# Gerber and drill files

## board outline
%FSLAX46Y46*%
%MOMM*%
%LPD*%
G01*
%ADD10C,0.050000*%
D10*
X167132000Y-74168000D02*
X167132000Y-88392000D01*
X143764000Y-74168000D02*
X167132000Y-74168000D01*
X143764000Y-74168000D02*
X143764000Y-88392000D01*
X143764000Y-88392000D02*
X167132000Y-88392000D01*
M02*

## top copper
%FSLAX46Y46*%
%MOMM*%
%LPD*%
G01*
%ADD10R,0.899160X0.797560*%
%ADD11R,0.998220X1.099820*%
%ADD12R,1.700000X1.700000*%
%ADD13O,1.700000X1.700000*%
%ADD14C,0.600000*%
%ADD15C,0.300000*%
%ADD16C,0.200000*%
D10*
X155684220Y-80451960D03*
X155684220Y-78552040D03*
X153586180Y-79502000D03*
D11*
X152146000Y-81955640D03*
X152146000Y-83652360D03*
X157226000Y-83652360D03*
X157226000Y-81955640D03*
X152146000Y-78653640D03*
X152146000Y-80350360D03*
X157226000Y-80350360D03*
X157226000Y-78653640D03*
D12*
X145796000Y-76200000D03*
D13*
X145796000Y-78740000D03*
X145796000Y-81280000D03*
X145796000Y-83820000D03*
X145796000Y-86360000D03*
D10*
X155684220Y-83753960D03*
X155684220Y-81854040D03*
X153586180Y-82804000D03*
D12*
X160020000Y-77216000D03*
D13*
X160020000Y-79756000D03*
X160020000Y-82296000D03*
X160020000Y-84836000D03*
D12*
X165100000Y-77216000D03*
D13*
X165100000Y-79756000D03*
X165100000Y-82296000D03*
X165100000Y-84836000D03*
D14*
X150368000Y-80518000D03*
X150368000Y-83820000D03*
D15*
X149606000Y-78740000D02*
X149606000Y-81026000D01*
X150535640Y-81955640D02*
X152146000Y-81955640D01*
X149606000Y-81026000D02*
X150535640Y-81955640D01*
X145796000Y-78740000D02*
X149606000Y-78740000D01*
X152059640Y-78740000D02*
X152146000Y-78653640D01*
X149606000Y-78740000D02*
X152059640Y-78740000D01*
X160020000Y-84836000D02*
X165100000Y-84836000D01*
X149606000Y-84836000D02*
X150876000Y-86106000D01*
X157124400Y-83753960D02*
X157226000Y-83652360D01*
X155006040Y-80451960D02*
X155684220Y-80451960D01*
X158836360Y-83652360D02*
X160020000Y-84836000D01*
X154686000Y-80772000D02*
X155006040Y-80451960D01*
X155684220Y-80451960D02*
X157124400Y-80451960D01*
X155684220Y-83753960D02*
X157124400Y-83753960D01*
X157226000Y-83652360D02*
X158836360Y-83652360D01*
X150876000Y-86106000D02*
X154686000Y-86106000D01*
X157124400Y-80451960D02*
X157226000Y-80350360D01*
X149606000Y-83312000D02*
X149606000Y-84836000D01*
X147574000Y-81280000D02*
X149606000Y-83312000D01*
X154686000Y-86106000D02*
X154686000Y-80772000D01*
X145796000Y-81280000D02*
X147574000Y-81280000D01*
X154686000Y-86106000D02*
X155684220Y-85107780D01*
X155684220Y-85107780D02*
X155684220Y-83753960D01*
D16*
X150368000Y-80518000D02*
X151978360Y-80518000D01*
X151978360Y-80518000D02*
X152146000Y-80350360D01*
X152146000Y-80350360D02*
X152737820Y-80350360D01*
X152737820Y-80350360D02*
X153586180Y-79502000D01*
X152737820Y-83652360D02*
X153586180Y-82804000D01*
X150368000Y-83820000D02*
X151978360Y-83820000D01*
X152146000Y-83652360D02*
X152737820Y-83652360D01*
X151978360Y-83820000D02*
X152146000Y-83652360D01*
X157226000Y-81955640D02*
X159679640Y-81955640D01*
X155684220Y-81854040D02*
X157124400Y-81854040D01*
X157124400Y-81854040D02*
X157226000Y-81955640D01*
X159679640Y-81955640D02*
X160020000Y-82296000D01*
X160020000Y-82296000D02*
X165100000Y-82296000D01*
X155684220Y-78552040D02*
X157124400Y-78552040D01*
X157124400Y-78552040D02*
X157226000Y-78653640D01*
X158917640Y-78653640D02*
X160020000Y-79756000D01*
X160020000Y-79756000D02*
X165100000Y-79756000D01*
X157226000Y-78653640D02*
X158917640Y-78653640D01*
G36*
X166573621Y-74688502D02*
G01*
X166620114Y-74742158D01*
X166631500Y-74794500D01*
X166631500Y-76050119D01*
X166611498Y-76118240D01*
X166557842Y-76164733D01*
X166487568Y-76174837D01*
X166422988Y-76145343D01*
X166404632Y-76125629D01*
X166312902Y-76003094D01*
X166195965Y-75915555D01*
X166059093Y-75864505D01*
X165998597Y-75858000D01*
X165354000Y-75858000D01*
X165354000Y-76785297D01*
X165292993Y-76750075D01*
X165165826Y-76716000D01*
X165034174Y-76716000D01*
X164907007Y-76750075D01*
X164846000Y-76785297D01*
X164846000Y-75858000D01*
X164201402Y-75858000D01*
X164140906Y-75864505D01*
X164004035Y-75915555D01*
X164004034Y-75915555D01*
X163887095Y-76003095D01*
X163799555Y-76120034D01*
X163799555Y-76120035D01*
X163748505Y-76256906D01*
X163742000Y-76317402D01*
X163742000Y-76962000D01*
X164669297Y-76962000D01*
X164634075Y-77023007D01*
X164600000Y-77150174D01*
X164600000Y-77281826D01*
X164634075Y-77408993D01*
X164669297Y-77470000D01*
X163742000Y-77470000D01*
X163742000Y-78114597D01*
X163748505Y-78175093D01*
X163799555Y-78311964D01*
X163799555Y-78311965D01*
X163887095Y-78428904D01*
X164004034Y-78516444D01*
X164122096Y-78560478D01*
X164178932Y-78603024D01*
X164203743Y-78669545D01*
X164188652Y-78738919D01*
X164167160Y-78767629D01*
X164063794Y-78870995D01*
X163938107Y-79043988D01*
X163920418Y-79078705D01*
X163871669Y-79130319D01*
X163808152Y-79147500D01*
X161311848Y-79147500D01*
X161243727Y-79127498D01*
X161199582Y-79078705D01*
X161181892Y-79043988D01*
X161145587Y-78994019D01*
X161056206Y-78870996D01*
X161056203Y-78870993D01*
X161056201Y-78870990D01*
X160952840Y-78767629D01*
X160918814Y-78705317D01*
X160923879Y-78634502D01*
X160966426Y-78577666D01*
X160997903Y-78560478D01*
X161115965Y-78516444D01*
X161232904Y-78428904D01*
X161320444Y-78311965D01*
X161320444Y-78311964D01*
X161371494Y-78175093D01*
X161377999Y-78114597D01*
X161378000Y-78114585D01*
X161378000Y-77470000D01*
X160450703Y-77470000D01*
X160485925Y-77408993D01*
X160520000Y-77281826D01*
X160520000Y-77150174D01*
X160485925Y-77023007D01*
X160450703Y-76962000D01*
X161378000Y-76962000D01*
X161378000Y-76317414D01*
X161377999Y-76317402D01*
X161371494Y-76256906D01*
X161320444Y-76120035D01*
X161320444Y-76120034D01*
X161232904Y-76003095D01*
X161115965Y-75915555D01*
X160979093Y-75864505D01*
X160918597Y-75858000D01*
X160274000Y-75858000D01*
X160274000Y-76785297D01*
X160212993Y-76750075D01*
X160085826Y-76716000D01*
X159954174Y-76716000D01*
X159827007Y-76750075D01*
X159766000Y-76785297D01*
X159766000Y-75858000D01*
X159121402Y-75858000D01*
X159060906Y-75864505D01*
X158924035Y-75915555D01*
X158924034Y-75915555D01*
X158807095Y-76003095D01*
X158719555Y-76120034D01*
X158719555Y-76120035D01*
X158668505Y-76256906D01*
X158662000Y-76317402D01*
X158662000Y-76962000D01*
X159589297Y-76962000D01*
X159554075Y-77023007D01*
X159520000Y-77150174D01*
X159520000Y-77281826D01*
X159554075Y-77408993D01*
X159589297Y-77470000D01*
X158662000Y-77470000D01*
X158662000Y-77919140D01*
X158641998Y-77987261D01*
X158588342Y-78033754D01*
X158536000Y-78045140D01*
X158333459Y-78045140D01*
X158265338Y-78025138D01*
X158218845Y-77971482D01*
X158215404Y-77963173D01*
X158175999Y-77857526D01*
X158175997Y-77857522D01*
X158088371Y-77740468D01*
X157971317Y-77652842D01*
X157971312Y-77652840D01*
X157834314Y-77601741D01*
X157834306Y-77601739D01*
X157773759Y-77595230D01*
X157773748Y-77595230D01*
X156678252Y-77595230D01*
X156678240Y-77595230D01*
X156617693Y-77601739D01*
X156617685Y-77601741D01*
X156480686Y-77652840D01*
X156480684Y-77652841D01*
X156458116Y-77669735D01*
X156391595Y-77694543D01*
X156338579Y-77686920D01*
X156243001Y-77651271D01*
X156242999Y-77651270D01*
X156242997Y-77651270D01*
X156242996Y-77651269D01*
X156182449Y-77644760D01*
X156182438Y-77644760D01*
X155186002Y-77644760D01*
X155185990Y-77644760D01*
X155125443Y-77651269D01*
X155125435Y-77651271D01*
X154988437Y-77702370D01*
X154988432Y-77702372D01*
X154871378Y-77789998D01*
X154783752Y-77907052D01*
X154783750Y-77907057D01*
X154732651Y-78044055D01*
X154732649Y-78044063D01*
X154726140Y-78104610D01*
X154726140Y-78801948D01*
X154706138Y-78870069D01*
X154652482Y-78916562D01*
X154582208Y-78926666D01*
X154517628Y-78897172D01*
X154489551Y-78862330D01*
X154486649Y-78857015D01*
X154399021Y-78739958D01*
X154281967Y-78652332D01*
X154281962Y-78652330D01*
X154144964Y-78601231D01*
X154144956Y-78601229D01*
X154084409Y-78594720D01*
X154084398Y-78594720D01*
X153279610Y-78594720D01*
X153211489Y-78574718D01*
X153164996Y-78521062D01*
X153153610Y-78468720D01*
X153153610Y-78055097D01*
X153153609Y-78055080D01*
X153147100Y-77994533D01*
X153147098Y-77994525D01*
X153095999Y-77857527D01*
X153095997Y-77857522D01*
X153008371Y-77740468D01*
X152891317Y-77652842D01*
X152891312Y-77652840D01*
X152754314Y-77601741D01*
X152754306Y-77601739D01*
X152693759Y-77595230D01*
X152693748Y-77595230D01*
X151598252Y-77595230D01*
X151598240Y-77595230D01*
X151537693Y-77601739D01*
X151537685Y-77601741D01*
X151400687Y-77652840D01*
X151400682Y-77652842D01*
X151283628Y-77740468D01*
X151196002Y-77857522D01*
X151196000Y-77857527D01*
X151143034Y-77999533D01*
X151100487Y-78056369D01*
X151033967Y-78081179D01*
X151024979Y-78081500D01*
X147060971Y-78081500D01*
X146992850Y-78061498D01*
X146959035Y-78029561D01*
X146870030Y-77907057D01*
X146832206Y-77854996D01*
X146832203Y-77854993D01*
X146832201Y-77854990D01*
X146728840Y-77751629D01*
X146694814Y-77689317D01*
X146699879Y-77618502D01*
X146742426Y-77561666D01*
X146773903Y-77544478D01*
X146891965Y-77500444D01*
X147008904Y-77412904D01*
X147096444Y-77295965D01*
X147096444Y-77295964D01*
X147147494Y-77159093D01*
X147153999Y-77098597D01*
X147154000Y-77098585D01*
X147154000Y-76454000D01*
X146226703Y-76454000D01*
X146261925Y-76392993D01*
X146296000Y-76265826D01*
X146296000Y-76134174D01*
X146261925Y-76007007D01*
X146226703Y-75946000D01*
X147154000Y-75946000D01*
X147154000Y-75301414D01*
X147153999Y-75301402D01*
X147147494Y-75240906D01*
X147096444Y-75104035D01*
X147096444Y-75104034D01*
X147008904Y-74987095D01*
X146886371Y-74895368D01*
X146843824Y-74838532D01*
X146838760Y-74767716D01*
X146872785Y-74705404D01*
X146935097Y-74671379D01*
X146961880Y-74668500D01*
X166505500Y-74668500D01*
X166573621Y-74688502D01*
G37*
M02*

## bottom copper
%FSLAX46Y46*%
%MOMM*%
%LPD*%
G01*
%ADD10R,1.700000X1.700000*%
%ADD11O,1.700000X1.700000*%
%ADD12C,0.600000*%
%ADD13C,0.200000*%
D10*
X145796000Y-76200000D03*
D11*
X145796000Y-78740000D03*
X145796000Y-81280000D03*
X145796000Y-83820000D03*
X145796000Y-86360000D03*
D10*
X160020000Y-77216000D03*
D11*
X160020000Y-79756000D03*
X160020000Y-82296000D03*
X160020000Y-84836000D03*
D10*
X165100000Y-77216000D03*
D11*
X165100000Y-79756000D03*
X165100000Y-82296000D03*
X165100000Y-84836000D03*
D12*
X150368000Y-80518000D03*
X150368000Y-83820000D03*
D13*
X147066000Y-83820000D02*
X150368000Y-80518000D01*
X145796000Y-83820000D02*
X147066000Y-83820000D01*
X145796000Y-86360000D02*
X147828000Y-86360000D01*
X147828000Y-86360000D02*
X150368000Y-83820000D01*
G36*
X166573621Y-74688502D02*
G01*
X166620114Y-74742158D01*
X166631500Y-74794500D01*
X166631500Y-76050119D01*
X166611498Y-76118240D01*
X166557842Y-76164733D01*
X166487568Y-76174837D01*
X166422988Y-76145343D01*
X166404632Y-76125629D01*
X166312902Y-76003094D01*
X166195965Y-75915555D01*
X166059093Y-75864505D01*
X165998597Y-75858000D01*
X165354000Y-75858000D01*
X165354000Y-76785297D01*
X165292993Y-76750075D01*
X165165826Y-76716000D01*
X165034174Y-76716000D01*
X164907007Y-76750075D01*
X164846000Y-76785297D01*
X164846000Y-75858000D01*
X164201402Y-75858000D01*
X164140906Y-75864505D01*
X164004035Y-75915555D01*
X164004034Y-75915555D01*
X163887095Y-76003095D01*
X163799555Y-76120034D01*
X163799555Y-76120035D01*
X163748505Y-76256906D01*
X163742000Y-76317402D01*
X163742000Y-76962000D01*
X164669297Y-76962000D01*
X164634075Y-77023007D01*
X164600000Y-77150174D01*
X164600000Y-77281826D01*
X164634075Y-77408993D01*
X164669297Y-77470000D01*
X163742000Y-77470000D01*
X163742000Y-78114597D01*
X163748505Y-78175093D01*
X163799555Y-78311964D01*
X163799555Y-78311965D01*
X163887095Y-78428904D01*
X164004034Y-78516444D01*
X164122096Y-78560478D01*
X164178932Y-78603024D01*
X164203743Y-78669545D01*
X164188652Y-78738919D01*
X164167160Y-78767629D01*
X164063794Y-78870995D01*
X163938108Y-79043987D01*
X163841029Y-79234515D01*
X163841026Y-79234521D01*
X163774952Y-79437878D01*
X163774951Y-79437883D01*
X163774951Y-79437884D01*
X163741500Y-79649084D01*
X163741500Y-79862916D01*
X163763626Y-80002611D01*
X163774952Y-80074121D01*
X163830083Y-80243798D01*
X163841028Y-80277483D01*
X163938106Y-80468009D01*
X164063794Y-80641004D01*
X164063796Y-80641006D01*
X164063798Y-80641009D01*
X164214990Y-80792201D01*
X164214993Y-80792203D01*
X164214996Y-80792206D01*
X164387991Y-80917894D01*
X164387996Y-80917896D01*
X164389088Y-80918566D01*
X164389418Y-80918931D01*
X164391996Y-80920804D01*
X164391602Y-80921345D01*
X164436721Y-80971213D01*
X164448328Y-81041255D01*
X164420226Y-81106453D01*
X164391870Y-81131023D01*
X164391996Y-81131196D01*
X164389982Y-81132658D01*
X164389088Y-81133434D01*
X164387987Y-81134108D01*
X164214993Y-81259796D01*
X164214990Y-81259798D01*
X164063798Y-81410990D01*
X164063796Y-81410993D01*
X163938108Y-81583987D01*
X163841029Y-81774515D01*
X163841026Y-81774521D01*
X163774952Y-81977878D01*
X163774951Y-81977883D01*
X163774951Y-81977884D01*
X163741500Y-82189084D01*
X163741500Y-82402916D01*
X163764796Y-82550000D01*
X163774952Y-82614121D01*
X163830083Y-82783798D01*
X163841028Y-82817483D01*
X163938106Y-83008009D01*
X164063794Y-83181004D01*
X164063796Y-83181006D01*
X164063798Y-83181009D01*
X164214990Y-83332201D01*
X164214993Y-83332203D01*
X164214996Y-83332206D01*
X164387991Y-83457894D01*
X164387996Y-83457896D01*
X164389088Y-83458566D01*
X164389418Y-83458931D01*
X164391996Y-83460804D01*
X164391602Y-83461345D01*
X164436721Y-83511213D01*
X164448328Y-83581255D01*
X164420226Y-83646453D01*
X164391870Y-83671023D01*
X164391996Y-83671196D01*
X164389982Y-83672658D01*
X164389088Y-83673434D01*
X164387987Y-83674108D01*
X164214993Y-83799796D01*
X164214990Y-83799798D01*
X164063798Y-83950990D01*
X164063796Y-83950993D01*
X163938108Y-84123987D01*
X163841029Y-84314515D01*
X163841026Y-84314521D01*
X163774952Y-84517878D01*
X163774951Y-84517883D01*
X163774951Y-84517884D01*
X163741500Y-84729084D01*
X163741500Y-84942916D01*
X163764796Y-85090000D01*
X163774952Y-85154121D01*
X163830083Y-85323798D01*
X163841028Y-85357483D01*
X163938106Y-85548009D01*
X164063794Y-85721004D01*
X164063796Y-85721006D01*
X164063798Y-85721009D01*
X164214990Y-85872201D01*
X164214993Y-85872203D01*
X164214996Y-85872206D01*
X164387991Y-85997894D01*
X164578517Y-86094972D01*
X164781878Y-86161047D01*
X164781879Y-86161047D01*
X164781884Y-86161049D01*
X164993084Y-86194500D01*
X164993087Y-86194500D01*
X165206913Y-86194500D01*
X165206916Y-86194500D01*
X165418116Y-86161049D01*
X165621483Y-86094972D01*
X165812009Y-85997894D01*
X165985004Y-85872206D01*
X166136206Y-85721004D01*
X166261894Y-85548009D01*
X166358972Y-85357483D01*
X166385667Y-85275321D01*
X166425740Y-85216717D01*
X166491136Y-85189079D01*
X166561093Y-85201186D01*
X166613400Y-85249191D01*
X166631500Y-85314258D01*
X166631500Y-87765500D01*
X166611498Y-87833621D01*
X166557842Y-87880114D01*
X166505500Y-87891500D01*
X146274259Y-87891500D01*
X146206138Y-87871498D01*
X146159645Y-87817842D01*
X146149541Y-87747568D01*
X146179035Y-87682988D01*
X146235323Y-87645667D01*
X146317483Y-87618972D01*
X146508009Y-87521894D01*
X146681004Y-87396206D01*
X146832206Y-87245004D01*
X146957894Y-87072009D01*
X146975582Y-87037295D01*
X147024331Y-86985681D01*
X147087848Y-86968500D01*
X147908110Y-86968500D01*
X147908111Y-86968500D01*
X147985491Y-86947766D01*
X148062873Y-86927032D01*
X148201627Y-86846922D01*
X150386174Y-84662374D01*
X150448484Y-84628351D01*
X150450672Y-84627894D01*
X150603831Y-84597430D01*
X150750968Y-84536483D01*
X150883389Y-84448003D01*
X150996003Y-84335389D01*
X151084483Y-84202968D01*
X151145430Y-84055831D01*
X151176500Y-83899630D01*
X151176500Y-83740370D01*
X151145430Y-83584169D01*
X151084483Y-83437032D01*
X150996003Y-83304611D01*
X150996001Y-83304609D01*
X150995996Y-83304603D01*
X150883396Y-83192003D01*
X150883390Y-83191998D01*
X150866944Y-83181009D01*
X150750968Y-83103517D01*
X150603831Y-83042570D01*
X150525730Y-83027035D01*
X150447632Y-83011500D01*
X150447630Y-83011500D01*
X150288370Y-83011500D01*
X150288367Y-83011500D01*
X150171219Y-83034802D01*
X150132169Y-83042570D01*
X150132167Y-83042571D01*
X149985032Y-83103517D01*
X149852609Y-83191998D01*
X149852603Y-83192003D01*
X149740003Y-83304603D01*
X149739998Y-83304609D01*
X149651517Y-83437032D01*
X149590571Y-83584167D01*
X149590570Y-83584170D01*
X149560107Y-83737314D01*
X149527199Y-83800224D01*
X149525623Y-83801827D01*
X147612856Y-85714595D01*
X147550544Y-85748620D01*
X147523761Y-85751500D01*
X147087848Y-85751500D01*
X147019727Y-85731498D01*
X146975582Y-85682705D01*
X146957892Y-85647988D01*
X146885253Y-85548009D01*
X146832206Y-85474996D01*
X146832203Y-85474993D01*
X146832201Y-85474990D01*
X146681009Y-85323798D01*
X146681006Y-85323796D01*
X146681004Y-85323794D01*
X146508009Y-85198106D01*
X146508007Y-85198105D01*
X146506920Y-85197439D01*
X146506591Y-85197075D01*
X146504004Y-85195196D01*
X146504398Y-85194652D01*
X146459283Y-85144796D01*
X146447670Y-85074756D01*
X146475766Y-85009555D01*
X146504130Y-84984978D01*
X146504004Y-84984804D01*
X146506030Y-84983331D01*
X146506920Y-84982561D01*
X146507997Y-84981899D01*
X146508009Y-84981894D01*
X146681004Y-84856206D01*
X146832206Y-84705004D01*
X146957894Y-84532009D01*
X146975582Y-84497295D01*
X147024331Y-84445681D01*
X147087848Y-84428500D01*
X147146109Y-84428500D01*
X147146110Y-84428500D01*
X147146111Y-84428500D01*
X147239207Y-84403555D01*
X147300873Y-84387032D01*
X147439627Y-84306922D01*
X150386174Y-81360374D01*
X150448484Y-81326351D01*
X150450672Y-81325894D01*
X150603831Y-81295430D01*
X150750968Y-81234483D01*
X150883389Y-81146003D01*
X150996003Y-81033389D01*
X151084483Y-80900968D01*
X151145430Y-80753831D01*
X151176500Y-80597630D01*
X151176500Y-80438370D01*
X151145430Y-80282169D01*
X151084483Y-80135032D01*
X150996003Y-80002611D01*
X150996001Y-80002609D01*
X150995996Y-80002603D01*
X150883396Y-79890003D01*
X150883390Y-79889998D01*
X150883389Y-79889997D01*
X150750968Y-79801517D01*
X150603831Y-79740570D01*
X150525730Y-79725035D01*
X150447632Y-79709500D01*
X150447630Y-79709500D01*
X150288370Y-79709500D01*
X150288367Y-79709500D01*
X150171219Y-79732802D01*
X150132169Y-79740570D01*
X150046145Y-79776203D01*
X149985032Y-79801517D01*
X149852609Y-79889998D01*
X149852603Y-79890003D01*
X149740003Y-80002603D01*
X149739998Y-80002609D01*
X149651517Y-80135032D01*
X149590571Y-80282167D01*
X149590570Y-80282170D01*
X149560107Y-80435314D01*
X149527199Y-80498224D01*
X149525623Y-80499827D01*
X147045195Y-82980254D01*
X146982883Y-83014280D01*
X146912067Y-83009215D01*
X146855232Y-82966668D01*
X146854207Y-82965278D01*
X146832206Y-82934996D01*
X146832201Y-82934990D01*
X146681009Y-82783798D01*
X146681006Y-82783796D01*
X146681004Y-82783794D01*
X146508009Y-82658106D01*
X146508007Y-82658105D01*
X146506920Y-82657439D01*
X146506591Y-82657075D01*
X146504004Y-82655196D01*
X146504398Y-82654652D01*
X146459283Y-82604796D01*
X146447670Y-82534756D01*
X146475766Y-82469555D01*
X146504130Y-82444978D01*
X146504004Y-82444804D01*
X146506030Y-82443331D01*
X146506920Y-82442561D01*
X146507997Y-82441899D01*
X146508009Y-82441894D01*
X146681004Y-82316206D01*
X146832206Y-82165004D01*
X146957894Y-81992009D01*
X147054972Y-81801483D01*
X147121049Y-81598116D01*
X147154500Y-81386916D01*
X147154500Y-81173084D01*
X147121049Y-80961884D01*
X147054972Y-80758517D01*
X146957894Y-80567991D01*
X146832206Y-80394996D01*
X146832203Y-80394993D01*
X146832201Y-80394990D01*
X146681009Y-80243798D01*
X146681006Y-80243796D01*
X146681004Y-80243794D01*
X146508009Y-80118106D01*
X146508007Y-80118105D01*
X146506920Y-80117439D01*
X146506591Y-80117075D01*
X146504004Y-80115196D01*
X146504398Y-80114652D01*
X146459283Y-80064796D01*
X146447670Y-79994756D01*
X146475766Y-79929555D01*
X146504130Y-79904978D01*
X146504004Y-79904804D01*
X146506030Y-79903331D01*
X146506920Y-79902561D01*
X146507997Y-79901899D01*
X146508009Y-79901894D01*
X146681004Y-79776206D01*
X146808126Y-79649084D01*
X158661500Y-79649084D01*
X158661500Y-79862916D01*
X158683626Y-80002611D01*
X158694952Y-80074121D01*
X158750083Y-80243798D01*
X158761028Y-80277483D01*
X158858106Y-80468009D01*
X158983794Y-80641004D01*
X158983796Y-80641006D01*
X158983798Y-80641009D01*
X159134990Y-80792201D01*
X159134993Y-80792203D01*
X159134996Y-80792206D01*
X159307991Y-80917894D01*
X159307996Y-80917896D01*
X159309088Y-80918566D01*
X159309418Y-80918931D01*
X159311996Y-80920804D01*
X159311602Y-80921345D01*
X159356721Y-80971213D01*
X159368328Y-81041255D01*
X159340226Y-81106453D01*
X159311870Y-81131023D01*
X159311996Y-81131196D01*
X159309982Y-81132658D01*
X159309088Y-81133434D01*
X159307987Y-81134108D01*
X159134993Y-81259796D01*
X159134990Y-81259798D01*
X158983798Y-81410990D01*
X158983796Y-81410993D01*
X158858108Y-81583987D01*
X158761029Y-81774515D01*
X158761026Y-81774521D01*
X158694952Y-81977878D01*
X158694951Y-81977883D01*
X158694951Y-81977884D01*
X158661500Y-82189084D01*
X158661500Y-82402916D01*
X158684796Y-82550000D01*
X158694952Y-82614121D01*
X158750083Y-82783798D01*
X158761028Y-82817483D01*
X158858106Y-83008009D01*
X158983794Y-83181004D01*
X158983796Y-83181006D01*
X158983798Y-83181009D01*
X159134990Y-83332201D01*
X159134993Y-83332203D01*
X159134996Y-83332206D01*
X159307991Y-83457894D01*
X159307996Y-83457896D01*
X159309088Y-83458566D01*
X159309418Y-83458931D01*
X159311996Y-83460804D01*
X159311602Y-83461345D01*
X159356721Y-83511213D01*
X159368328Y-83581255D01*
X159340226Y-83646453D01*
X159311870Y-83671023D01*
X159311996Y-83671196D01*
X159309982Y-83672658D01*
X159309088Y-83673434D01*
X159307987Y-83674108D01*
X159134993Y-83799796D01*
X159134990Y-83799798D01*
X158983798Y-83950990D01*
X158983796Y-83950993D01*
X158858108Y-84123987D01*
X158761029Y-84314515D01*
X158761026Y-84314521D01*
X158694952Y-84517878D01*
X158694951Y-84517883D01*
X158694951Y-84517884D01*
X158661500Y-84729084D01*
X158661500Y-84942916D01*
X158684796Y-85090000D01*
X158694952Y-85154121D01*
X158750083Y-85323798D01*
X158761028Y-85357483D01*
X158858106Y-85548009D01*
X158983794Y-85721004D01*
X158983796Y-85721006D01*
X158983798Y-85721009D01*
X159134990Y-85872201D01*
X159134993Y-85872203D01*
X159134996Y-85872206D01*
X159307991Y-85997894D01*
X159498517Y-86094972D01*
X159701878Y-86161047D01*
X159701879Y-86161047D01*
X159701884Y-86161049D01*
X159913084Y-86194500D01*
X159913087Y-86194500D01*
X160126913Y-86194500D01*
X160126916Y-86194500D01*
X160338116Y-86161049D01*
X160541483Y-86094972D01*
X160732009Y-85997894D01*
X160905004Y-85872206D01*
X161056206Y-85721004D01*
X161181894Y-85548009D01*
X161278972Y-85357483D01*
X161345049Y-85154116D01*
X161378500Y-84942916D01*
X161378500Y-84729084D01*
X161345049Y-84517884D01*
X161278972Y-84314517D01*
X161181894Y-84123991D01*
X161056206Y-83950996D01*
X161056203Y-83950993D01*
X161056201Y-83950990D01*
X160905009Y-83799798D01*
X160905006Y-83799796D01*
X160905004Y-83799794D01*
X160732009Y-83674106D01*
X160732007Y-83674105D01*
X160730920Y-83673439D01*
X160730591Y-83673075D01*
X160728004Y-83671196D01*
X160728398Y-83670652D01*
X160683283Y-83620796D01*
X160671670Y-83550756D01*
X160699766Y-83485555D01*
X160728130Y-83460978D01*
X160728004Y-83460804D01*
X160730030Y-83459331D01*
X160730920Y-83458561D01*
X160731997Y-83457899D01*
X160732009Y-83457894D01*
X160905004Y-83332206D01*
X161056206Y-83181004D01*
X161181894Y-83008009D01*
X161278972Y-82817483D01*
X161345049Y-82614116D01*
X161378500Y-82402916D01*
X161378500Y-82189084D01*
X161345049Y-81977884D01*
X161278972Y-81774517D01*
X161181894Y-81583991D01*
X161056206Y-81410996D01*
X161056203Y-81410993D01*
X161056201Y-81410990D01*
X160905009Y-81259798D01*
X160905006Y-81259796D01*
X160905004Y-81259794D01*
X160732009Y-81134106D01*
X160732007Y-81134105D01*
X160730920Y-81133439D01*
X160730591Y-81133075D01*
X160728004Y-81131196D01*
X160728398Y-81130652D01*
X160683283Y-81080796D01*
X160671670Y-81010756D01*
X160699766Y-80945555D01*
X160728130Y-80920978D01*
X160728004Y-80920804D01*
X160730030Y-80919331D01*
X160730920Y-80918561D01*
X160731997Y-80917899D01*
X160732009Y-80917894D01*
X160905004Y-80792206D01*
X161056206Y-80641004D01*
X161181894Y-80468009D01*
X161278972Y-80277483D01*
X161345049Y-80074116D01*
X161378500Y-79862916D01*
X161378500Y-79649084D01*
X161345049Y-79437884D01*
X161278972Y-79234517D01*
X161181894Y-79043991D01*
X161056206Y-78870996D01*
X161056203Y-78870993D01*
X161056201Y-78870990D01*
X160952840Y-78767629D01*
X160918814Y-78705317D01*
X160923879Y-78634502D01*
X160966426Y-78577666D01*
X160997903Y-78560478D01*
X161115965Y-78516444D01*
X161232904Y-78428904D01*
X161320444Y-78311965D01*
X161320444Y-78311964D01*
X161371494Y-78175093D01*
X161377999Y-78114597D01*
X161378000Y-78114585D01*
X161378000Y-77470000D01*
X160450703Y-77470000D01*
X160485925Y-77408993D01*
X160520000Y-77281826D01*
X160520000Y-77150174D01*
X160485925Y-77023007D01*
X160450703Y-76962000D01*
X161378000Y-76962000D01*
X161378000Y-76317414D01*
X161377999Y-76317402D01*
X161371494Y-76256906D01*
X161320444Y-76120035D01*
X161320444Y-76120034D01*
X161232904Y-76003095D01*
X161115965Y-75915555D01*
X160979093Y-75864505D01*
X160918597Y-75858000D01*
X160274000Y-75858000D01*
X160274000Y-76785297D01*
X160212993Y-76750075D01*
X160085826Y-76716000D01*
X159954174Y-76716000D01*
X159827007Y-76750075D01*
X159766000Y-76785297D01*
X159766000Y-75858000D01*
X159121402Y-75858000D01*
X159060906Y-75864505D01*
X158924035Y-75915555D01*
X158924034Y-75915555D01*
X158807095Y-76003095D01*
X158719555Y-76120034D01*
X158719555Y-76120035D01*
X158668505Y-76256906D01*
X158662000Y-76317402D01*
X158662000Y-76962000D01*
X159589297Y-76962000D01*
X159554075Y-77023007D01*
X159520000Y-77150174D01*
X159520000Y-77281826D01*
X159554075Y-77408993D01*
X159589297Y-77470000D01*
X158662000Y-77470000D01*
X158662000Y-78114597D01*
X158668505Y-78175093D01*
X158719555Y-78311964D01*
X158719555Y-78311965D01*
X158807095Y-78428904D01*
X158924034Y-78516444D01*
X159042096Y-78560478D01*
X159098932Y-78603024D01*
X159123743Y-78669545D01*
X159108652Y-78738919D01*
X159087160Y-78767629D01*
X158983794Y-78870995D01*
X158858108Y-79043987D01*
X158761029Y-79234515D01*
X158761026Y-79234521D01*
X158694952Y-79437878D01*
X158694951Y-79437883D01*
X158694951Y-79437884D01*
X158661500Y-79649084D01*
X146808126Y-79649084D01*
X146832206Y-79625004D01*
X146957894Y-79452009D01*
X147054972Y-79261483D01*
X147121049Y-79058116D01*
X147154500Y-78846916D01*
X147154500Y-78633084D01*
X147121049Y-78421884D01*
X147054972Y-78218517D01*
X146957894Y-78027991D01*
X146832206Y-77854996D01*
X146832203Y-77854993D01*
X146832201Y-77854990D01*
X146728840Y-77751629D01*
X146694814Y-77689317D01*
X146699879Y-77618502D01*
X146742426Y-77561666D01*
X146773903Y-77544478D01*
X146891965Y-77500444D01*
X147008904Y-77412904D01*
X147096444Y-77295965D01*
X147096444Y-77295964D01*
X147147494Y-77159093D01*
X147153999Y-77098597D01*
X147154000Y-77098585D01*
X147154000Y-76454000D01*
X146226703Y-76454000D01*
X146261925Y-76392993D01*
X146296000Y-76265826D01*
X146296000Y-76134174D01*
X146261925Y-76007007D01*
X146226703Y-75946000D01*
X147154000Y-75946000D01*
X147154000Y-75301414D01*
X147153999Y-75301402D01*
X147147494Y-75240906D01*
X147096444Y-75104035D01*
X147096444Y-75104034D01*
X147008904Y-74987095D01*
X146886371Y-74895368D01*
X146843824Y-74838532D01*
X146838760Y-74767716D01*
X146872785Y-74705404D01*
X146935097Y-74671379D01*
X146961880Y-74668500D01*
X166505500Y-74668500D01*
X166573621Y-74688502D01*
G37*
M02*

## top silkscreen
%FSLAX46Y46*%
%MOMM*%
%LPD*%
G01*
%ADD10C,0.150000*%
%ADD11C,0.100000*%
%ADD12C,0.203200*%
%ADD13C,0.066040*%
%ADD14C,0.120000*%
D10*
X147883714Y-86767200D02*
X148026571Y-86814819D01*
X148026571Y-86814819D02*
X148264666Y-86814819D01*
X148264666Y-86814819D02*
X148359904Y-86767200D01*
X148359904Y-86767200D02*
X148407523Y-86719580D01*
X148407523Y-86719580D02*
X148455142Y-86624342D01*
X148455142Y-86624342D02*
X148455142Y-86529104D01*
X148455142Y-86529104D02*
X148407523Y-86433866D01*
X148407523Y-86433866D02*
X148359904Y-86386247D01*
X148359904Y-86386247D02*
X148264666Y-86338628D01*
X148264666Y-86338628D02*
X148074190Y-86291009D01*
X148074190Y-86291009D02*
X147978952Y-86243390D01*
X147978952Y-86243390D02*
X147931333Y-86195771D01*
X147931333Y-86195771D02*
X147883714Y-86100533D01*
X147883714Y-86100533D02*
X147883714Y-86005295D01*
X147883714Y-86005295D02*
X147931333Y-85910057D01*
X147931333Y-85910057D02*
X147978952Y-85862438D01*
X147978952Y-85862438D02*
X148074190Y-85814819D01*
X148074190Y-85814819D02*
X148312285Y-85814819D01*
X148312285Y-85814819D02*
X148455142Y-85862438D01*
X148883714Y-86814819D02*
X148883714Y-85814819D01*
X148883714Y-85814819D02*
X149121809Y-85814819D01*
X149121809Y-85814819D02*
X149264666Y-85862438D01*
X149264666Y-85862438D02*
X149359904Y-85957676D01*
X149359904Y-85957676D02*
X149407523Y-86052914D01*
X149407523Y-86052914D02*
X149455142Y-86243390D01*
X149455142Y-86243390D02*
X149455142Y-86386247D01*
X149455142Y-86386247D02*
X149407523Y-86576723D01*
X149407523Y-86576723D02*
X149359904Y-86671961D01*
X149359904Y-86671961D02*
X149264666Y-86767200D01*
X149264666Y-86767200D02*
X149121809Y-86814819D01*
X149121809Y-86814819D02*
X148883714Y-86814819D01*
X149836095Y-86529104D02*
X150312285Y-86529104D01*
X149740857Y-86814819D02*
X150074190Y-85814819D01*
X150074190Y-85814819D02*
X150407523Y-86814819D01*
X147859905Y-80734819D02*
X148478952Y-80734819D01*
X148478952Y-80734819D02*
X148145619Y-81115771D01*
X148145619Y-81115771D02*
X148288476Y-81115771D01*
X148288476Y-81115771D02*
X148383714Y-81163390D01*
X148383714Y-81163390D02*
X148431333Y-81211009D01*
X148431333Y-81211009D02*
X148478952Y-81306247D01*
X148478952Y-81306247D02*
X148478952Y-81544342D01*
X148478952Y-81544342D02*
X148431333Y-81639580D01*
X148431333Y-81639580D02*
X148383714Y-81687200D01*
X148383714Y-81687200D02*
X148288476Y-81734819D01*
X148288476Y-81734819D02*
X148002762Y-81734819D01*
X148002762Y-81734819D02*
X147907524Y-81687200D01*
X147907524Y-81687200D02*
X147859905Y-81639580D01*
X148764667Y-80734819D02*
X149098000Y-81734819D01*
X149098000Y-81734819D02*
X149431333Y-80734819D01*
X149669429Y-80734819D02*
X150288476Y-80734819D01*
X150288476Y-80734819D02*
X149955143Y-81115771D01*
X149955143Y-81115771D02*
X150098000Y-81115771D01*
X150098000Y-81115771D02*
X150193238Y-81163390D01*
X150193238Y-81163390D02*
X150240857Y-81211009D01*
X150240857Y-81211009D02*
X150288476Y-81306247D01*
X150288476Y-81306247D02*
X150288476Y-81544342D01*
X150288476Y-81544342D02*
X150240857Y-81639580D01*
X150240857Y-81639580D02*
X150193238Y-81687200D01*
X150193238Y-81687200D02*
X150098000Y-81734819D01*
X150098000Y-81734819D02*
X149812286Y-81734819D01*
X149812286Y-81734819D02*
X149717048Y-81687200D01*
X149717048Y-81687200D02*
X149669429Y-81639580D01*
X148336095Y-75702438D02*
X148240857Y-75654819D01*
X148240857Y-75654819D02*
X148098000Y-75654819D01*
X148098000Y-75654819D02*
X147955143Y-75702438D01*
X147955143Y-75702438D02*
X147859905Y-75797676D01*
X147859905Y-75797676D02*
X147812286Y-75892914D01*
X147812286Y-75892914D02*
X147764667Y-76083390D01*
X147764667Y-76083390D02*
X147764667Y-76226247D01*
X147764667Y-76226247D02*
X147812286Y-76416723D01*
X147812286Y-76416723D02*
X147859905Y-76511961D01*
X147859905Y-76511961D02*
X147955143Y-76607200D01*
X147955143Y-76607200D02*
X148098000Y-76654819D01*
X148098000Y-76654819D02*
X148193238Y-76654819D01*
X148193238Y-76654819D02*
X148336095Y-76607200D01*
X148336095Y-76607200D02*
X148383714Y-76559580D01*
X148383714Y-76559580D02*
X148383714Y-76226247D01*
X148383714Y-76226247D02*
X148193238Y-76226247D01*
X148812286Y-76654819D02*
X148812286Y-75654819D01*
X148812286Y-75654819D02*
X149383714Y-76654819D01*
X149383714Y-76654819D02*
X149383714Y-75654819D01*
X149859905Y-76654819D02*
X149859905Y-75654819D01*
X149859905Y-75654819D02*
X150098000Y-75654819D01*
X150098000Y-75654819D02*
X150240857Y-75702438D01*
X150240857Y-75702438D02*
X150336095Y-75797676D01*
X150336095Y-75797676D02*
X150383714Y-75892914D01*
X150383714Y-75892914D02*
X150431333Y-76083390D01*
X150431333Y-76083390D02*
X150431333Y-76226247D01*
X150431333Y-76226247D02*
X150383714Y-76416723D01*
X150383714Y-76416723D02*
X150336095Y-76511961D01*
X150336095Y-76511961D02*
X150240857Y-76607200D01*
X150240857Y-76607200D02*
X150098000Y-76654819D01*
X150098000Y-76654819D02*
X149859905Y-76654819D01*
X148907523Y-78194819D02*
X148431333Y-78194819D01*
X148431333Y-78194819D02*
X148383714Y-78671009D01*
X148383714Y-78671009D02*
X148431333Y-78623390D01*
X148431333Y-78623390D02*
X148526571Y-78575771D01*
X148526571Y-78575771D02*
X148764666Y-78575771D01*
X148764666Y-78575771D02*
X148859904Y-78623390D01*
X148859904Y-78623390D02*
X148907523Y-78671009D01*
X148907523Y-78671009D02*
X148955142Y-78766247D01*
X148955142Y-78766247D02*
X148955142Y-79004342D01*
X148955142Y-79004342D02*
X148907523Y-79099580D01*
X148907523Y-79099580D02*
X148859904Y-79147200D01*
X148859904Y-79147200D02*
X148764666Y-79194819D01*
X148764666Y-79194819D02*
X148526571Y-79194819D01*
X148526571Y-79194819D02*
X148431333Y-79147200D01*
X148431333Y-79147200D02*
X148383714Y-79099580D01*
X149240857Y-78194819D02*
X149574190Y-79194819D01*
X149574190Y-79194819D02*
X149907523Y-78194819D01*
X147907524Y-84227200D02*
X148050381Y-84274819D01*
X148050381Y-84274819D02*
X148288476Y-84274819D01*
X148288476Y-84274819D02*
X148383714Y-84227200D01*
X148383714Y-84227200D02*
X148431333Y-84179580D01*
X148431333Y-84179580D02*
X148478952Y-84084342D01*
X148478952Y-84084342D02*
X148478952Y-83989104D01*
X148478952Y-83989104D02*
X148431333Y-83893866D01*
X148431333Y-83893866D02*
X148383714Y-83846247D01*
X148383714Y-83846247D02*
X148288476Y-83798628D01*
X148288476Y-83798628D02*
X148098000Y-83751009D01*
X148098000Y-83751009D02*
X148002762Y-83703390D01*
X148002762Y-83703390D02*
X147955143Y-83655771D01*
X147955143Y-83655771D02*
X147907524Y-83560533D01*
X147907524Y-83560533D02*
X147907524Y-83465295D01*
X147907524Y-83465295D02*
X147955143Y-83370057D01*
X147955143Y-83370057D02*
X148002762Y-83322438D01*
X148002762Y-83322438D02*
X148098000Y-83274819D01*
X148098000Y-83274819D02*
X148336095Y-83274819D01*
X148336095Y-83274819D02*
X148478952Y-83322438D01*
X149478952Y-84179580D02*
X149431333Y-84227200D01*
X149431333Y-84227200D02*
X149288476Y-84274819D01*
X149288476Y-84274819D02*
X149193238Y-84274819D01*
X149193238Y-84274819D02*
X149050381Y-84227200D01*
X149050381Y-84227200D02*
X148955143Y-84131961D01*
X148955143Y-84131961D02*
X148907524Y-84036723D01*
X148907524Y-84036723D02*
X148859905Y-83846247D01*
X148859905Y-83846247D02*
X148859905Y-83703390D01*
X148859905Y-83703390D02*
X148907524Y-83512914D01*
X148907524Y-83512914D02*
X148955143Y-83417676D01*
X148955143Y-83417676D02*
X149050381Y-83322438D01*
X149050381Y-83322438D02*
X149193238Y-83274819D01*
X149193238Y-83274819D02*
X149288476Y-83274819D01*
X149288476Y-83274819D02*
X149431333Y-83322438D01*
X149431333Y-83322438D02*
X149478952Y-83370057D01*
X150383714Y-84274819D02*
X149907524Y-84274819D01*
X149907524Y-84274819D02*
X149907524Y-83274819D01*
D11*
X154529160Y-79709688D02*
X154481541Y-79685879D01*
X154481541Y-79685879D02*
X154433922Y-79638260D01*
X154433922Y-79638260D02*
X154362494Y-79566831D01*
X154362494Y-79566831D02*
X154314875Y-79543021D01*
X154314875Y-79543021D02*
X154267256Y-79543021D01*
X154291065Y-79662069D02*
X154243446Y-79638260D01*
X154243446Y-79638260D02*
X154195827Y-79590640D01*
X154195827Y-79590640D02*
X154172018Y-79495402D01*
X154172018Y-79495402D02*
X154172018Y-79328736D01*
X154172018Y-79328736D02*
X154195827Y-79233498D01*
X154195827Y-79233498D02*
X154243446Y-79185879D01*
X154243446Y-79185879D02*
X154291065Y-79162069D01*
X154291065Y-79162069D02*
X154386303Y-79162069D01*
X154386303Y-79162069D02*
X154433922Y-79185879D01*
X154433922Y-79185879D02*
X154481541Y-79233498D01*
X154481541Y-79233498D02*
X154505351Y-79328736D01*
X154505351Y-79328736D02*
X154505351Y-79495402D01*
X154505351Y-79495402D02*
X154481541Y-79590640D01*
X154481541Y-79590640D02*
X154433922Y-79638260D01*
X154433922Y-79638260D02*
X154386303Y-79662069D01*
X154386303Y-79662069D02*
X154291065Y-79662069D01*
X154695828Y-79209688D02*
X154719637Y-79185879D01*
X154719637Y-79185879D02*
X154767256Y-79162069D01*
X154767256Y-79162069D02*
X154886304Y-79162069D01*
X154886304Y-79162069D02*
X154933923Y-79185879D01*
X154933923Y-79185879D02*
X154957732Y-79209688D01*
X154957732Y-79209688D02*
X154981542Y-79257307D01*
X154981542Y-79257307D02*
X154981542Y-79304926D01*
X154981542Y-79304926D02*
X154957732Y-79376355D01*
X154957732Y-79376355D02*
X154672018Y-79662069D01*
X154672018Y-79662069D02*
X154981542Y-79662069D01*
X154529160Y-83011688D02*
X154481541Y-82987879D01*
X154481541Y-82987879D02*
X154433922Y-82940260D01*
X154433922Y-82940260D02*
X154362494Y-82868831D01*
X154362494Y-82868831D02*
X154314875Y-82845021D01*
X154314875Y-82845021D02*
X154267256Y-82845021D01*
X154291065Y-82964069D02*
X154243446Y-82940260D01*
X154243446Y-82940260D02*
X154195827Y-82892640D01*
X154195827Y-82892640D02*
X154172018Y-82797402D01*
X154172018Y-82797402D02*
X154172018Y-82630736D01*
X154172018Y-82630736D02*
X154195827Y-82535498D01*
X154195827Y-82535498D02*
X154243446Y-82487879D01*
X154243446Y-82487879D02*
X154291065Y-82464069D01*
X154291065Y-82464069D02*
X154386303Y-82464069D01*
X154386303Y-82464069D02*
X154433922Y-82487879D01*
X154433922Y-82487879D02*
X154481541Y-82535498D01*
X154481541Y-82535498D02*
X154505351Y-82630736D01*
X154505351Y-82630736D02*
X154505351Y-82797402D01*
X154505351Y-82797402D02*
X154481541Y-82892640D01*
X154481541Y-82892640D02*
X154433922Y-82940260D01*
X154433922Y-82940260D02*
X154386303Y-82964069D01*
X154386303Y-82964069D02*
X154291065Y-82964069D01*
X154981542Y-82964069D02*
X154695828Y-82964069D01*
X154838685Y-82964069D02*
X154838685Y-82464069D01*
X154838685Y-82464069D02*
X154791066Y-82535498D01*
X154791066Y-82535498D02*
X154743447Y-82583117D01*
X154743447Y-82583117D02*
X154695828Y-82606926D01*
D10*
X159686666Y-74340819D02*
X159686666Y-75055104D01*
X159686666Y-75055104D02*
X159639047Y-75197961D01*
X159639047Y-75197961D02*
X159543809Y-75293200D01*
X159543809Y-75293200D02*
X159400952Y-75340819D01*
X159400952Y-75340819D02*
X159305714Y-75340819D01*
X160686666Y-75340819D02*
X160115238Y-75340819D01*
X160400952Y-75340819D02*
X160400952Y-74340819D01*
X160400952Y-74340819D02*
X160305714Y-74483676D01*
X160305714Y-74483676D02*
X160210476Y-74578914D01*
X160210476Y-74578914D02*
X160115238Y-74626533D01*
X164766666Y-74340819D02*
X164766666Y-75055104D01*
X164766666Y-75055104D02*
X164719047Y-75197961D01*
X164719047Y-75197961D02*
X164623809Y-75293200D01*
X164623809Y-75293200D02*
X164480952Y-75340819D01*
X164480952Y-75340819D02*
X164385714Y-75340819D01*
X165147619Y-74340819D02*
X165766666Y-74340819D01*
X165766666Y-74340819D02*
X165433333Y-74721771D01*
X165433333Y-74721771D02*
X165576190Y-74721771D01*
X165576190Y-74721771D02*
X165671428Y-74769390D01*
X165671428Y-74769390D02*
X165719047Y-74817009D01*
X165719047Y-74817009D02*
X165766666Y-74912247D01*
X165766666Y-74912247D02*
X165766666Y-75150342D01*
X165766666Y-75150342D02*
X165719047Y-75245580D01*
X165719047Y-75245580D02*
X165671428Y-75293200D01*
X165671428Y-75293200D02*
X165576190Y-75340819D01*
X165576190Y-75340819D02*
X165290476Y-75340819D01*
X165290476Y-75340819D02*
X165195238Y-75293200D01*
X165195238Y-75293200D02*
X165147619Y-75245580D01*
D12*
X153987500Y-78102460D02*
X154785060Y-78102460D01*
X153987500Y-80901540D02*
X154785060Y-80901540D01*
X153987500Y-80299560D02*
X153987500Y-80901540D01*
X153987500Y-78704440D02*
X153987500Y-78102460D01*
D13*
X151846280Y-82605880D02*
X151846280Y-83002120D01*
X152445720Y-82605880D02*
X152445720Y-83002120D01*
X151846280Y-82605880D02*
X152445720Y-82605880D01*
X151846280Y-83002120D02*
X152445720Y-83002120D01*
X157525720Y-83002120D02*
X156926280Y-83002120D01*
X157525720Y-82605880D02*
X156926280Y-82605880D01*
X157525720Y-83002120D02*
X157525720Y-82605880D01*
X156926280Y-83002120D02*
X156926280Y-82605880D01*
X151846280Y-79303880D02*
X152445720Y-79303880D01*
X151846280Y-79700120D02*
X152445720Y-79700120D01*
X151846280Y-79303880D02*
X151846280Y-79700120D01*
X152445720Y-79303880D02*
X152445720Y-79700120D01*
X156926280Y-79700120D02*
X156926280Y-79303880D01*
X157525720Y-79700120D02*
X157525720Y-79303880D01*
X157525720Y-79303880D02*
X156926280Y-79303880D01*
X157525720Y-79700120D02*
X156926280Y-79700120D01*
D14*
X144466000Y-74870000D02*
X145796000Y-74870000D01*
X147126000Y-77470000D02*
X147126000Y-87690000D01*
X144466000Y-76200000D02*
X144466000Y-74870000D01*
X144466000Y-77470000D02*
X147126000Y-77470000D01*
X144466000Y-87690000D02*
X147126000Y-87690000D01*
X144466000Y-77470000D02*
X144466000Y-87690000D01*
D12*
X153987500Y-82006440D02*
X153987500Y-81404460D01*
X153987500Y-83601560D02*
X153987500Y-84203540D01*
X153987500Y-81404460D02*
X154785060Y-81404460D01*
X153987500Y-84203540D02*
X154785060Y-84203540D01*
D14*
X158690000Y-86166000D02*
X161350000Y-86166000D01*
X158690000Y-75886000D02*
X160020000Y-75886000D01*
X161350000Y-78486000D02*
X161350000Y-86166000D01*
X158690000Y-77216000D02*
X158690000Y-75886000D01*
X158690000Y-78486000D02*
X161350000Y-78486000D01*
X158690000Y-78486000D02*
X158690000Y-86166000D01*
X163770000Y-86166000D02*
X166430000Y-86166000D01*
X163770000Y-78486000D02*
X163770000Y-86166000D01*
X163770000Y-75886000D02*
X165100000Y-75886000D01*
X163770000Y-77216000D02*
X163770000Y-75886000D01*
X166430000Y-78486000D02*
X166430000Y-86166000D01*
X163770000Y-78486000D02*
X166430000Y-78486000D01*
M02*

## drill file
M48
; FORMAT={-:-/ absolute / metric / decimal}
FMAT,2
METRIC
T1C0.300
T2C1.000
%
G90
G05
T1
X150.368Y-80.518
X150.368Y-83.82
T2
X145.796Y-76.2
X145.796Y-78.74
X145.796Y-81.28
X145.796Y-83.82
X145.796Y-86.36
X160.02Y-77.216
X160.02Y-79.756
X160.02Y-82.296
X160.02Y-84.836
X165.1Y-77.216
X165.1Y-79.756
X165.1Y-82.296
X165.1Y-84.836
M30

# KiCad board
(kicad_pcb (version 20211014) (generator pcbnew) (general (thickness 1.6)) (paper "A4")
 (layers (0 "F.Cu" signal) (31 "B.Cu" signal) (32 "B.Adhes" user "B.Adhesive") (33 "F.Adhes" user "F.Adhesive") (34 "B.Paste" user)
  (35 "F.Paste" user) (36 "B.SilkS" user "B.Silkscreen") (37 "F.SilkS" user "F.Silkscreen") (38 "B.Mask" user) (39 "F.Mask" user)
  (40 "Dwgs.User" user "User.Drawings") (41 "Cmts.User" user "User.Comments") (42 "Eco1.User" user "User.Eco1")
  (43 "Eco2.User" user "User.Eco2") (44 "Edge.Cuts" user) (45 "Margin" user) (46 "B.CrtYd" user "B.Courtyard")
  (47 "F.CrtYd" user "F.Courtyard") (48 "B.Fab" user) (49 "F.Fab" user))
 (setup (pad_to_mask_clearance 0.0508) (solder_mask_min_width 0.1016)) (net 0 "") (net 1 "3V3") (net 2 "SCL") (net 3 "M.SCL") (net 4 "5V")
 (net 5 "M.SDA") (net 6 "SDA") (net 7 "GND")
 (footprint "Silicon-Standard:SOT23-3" (layer "F.Cu") (at 154.686 79.502 90)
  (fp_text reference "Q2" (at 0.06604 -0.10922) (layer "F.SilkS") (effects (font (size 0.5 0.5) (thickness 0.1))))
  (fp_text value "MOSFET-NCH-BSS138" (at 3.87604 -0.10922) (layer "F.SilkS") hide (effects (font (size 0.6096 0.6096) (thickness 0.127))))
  (fp_line (start 1.39954 -0.6985) (end 1.39954 0.09906) (layer "F.SilkS") (width 0.2032))
  (fp_line (start -1.39954 -0.6985) (end -1.39954 0.09906) (layer "F.SilkS") (width 0.2032))
  (fp_line (start -0.79756 -0.6985) (end -1.39954 -0.6985) (layer "F.SilkS") (width 0.2032))
  (fp_line (start 0.79756 -0.6985) (end 1.39954 -0.6985) (layer "F.SilkS") (width 0.2032))
  (pad "1" smd rect locked (at -0.94996 0.99822 90) (size 0.79756 0.89916) (layers "F.Cu" "F.Paste" "F.Mask") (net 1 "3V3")
   (solder_mask_margin 0.1016))
  (pad "2" smd rect locked (at 0.94996 0.99822 90) (size 0.79756 0.89916) (layers "F.Cu" "F.Paste" "F.Mask") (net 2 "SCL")
   (solder_mask_margin 0.1016))
  (pad "3" smd rect locked (at 0 -1.09982 90) (size 0.79756 0.89916) (layers "F.Cu" "F.Paste" "F.Mask") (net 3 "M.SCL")
   (solder_mask_margin 0.1016)))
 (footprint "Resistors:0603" (layer "F.Cu") (at 152.146 82.804 -90)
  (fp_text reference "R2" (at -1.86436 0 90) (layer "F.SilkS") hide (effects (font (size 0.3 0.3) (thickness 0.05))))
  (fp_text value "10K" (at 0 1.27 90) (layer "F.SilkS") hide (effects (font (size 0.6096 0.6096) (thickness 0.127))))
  (fp_line (start -0.19812 0.29972) (end 0.19812 0.29972) (layer "F.SilkS") (width 0.06604))
  (fp_line (start -0.19812 -0.29972) (end 0.19812 -0.29972) (layer "F.SilkS") (width 0.06604))
  (fp_line (start -0.19812 0.29972) (end -0.19812 -0.29972) (layer "F.SilkS") (width 0.06604))
  (fp_line (start 0.19812 0.29972) (end 0.19812 -0.29972) (layer "F.SilkS") (width 0.06604))
  (pad "1" smd rect locked (at -0.84836 0 270) (size 1.09982 0.99822) (layers "F.Cu" "F.Paste" "F.Mask") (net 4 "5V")
   (solder_mask_margin 0.1016))
  (pad "2" smd rect locked (at 0.84836 0 270) (size 1.09982 0.99822) (layers "F.Cu" "F.Paste" "F.Mask") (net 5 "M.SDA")
   (solder_mask_margin 0.1016)))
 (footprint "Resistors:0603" (layer "F.Cu") (at 157.226 82.804 90)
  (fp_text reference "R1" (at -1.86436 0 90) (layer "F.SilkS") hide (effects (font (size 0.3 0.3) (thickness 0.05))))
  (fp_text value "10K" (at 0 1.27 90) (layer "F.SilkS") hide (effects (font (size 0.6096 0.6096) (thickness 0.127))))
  (fp_line (start -0.19812 0.29972) (end -0.19812 -0.29972) (layer "F.SilkS") (width 0.06604))
  (fp_line (start 0.19812 0.29972) (end 0.19812 -0.29972) (layer "F.SilkS") (width 0.06604))
  (fp_line (start -0.19812 0.29972) (end 0.19812 0.29972) (layer "F.SilkS") (width 0.06604))
  (fp_line (start -0.19812 -0.29972) (end 0.19812 -0.29972) (layer "F.SilkS") (width 0.06604))
  (pad "1" smd rect locked (at -0.84836 0 90) (size 1.09982 0.99822) (layers "F.Cu" "F.Paste" "F.Mask") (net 1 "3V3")
   (solder_mask_margin 0.1016))
  (pad "2" smd rect locked (at 0.84836 0 90) (size 1.09982 0.99822) (layers "F.Cu" "F.Paste" "F.Mask") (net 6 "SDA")
   (solder_mask_margin 0.1016)))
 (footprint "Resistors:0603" (layer "F.Cu") (at 152.146 79.502 -90)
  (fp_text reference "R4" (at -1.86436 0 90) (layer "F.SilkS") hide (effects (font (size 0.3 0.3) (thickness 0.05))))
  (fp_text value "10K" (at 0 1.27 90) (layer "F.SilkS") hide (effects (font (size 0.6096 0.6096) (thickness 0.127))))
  (fp_line (start -0.19812 0.29972) (end -0.19812 -0.29972) (layer "F.SilkS") (width 0.06604))
  (fp_line (start 0.19812 0.29972) (end 0.19812 -0.29972) (layer "F.SilkS") (width 0.06604))
  (fp_line (start -0.19812 0.29972) (end 0.19812 0.29972) (layer "F.SilkS") (width 0.06604))
  (fp_line (start -0.19812 -0.29972) (end 0.19812 -0.29972) (layer "F.SilkS") (width 0.06604))
  (pad "1" smd rect locked (at -0.84836 0 270) (size 1.09982 0.99822) (layers "F.Cu" "F.Paste" "F.Mask") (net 4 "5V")
   (solder_mask_margin 0.1016))
  (pad "2" smd rect locked (at 0.84836 0 270) (size 1.09982 0.99822) (layers "F.Cu" "F.Paste" "F.Mask") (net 3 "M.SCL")
   (solder_mask_margin 0.1016)))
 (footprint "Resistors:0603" (layer "F.Cu") (at 157.226 79.502 90)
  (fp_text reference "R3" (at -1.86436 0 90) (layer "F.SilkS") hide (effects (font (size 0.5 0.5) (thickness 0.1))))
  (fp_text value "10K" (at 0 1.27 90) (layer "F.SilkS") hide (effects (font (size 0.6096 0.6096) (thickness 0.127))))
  (fp_line (start -0.19812 -0.29972) (end 0.19812 -0.29972) (layer "F.SilkS") (width 0.06604))
  (fp_line (start -0.19812 0.29972) (end 0.19812 0.29972) (layer "F.SilkS") (width 0.06604))
  (fp_line (start 0.19812 0.29972) (end 0.19812 -0.29972) (layer "F.SilkS") (width 0.06604))
  (fp_line (start -0.19812 0.29972) (end -0.19812 -0.29972) (layer "F.SilkS") (width 0.06604))
  (pad "1" smd rect locked (at -0.84836 0 90) (size 1.09982 0.99822) (layers "F.Cu" "F.Paste" "F.Mask") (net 1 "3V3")
   (solder_mask_margin 0.1016))
  (pad "2" smd rect locked (at 0.84836 0 90) (size 1.09982 0.99822) (layers "F.Cu" "F.Paste" "F.Mask") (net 2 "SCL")
   (solder_mask_margin 0.1016)))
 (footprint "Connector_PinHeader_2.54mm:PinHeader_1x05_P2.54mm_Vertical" (layer "F.Cu") (at 145.796 76.2)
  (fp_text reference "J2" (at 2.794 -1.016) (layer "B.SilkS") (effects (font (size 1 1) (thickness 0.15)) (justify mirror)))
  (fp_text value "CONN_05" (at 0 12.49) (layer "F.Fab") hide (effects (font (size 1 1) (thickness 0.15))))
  (fp_line (start -1.33 -1.33) (end 0 -1.33) (layer "F.SilkS") (width 0.12))
  (fp_line (start 1.33 1.27) (end 1.33 11.49) (layer "F.SilkS") (width 0.12))
  (fp_line (start -1.33 0) (end -1.33 -1.33) (layer "F.SilkS") (width 0.12))
  (fp_line (start -1.33 1.27) (end 1.33 1.27) (layer "F.SilkS") (width 0.12))
  (fp_line (start -1.33 11.49) (end 1.33 11.49) (layer "F.SilkS") (width 0.12))
  (fp_line (start -1.33 1.27) (end -1.33 11.49) (layer "F.SilkS") (width 0.12))
  (pad "1" thru_hole rect locked (at 0 0) (size 1.7 1.7) (drill 1) (layers *.Cu *.Mask) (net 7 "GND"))
  (pad "2" thru_hole oval locked (at 0 2.54) (size 1.7 1.7) (drill 1) (layers *.Cu *.Mask) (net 4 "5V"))
  (pad "3" thru_hole oval locked (at 0 5.08) (size 1.7 1.7) (drill 1) (layers *.Cu *.Mask) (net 1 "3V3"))
  (pad "4" thru_hole oval locked (at 0 7.62) (size 1.7 1.7) (drill 1) (layers *.Cu *.Mask) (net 3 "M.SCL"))
  (pad "5" thru_hole oval locked (at 0 10.16) (size 1.7 1.7) (drill 1) (layers *.Cu *.Mask) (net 5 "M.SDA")))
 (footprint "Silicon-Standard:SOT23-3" (layer "F.Cu") (at 154.686 82.804 90)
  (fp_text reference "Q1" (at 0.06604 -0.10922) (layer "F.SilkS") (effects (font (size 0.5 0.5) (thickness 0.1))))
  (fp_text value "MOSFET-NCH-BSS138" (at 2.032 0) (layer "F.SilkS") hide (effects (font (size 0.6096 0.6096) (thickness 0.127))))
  (fp_line (start 0.79756 -0.6985) (end 1.39954 -0.6985) (layer "F.SilkS") (width 0.2032))
  (fp_line (start -0.79756 -0.6985) (end -1.39954 -0.6985) (layer "F.SilkS") (width 0.2032))
  (fp_line (start 1.39954 -0.6985) (end 1.39954 0.09906) (layer "F.SilkS") (width 0.2032))
  (fp_line (start -1.39954 -0.6985) (end -1.39954 0.09906) (layer "F.SilkS") (width 0.2032))
  (pad "1" smd rect locked (at -0.94996 0.99822 90) (size 0.79756 0.89916) (layers "F.Cu" "F.Paste" "F.Mask") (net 1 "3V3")
   (solder_mask_margin 0.1016))
  (pad "2" smd rect locked (at 0.94996 0.99822 90) (size 0.79756 0.89916) (layers "F.Cu" "F.Paste" "F.Mask") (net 6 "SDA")
   (solder_mask_margin 0.1016))
  (pad "3" smd rect locked (at 0 -1.09982 90) (size 0.79756 0.89916) (layers "F.Cu" "F.Paste" "F.Mask") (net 5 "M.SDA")
   (solder_mask_margin 0.1016)))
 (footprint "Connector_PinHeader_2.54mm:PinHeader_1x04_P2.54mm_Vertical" (layer "F.Cu") (at 160.02 77.216)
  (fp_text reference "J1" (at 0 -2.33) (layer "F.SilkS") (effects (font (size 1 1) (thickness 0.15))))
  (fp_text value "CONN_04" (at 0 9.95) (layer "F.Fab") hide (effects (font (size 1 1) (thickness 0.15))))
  (fp_line (start -1.33 8.95) (end 1.33 8.95) (layer "F.SilkS") (width 0.12))
  (fp_line (start -1.33 -1.33) (end 0 -1.33) (layer "F.SilkS") (width 0.12))
  (fp_line (start 1.33 1.27) (end 1.33 8.95) (layer "F.SilkS") (width 0.12))
  (fp_line (start -1.33 0) (end -1.33 -1.33) (layer "F.SilkS") (width 0.12))
  (fp_line (start -1.33 1.27) (end 1.33 1.27) (layer "F.SilkS") (width 0.12))
  (fp_line (start -1.33 1.27) (end -1.33 8.95) (layer "F.SilkS") (width 0.12))
  (pad "1" thru_hole rect locked (at 0 0) (size 1.7 1.7) (drill 1) (layers *.Cu *.Mask) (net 7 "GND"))
  (pad "2" thru_hole oval locked (at 0 2.54) (size 1.7 1.7) (drill 1) (layers *.Cu *.Mask) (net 2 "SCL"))
  (pad "3" thru_hole oval locked (at 0 5.08) (size 1.7 1.7) (drill 1) (layers *.Cu *.Mask) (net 6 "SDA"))
  (pad "4" thru_hole oval locked (at 0 7.62) (size 1.7 1.7) (drill 1) (layers *.Cu *.Mask) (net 1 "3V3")))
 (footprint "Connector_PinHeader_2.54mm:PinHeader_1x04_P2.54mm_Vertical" (layer "F.Cu") (at 165.1 77.216)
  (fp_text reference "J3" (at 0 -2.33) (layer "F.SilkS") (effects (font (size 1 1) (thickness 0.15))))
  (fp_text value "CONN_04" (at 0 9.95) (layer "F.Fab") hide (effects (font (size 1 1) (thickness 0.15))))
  (fp_line (start -1.33 8.95) (end 1.33 8.95) (layer "F.SilkS") (width 0.12))
  (fp_line (start -1.33 1.27) (end -1.33 8.95) (layer "F.SilkS") (width 0.12))
  (fp_line (start -1.33 -1.33) (end 0 -1.33) (layer "F.SilkS") (width 0.12))
  (fp_line (start -1.33 0) (end -1.33 -1.33) (layer "F.SilkS") (width 0.12))
  (fp_line (start 1.33 1.27) (end 1.33 8.95) (layer "F.SilkS") (width 0.12))
  (fp_line (start -1.33 1.27) (end 1.33 1.27) (layer "F.SilkS") (width 0.12))
  (pad "1" thru_hole rect locked (at 0 0) (size 1.7 1.7) (drill 1) (layers *.Cu *.Mask) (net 7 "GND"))
  (pad "2" thru_hole oval locked (at 0 2.54) (size 1.7 1.7) (drill 1) (layers *.Cu *.Mask) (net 2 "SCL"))
  (pad "3" thru_hole oval locked (at 0 5.08) (size 1.7 1.7) (drill 1) (layers *.Cu *.Mask) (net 6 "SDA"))
  (pad "4" thru_hole oval locked (at 0 7.62) (size 1.7 1.7) (drill 1) (layers *.Cu *.Mask) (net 1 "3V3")))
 (gr_line (start 167.132 74.168) (end 167.132 88.392) (layer "Edge.Cuts") (width 0.05))
 (gr_line (start 143.764 74.168) (end 167.132 74.168) (layer "Edge.Cuts") (width 0.05))
 (gr_line (start 143.764 74.168) (end 143.764 88.392) (layer "Edge.Cuts") (width 0.05))
 (gr_line (start 143.764 88.392) (end 167.132 88.392) (layer "Edge.Cuts") (width 0.05))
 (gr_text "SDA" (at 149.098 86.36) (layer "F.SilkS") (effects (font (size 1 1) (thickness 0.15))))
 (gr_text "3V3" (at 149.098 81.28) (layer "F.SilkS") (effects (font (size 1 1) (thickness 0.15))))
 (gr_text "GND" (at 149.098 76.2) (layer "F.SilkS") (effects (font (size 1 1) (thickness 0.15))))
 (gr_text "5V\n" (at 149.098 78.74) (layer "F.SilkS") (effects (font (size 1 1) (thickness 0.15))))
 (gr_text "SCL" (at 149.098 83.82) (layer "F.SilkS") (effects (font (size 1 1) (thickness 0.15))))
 (segment (start 149.606 78.74) (end 149.606 81.026) (width 0.3) (layer "F.Cu") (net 4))
 (segment (start 150.53564 81.95564) (end 152.146 81.95564) (width 0.3) (layer "F.Cu") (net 4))
 (segment (start 149.606 81.026) (end 150.53564 81.95564) (width 0.3) (layer "F.Cu") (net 4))
 (segment (start 145.796 78.74) (end 149.606 78.74) (width 0.3) (layer "F.Cu") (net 4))
 (segment (start 152.05964 78.74) (end 152.146 78.65364) (width 0.3) (layer "F.Cu") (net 4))
 (segment (start 149.606 78.74) (end 152.05964 78.74) (width 0.3) (layer "F.Cu") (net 4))
 (segment (start 160.02 84.836) (end 165.1 84.836) (width 0.3) (layer "F.Cu") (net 1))
 (segment (start 149.606 84.836) (end 150.876 86.106) (width 0.3) (layer "F.Cu") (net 1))
 (segment (start 157.1244 83.75396) (end 157.226 83.65236) (width 0.3) (layer "F.Cu") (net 1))
 (segment (start 155.00604 80.45196) (end 155.68422 80.45196) (width 0.3) (layer "F.Cu") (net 1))
 (segment (start 158.83636 83.65236) (end 160.02 84.836) (width 0.3) (layer "F.Cu") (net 1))
 (segment (start 154.686 80.772) (end 155.00604 80.45196) (width 0.3) (layer "F.Cu") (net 1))
 (segment (start 155.68422 80.45196) (end 157.1244 80.45196) (width 0.3) (layer "F.Cu") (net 1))
 (segment (start 155.68422 83.75396) (end 157.1244 83.75396) (width 0.3) (layer "F.Cu") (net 1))
 (segment (start 157.226 83.65236) (end 158.83636 83.65236) (width 0.3) (layer "F.Cu") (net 1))
 (segment (start 150.876 86.106) (end 154.686 86.106) (width 0.3) (layer "F.Cu") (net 1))
 (segment (start 157.1244 80.45196) (end 157.226 80.35036) (width 0.3) (layer "F.Cu") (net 1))
 (segment (start 149.606 83.312) (end 149.606 84.836) (width 0.3) (layer "F.Cu") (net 1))
 (segment (start 147.574 81.28) (end 149.606 83.312) (width 0.3) (layer "F.Cu") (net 1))
 (segment (start 154.686 86.106) (end 154.686 80.772) (width 0.3) (layer "F.Cu") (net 1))
 (segment (start 145.796 81.28) (end 147.574 81.28) (width 0.3) (layer "F.Cu") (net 1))
 (segment (start 154.686 86.106) (end 155.68422 85.10778) (width 0.3) (layer "F.Cu") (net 1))
 (segment (start 155.68422 85.10778) (end 155.68422 83.75396) (width 0.3) (layer "F.Cu") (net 1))
 (segment (start 150.368 80.518) (end 151.97836 80.518) (width 0.2) (layer "F.Cu") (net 3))
 (segment (start 151.97836 80.518) (end 152.146 80.35036) (width 0.2) (layer "F.Cu") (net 3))
 (segment (start 152.146 80.35036) (end 152.73782 80.35036) (width 0.2) (layer "F.Cu") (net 3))
 (segment (start 152.73782 80.35036) (end 153.58618 79.502) (width 0.2) (layer "F.Cu") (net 3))
 (via (at 150.368 80.518) (size 0.6) (drill 0.3) (layers "F.Cu" "B.Cu") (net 3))
 (segment (start 147.066 83.82) (end 150.368 80.518) (width 0.2) (layer "B.Cu") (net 3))
 (segment (start 145.796 83.82) (end 147.066 83.82) (width 0.2) (layer "B.Cu") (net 3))
 (segment (start 152.73782 83.65236) (end 153.58618 82.804) (width 0.2) (layer "F.Cu") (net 5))
 (segment (start 150.368 83.82) (end 151.97836 83.82) (width 0.2) (layer "F.Cu") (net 5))
 (segment (start 152.146 83.65236) (end 152.73782 83.65236) (width 0.2) (layer "F.Cu") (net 5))
 (segment (start 151.97836 83.82) (end 152.146 83.65236) (width 0.2) (layer "F.Cu") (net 5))
 (via (at 150.368 83.82) (size 0.6) (drill 0.3) (layers "F.Cu" "B.Cu") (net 5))
 (segment (start 145.796 86.36) (end 147.828 86.36) (width 0.2) (layer "B.Cu") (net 5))
 (segment (start 147.828 86.36) (end 150.368 83.82) (width 0.2) (layer "B.Cu") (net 5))
 (segment (start 157.226 81.95564) (end 159.67964 81.95564) (width 0.2) (layer "F.Cu") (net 6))
 (segment (start 155.68422 81.85404) (end 157.1244 81.85404) (width 0.2) (layer "F.Cu") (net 6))
 (segment (start 157.1244 81.85404) (end 157.226 81.95564) (width 0.2) (layer "F.Cu") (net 6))
 (segment (start 159.67964 81.95564) (end 160.02 82.296) (width 0.2) (layer "F.Cu") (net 6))
 (segment (start 160.02 82.296) (end 165.1 82.296) (width 0.2) (layer "F.Cu") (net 6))
 (segment (start 155.68422 78.55204) (end 157.1244 78.55204) (width 0.2) (layer "F.Cu") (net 2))
 (segment (start 157.1244 78.55204) (end 157.226 78.65364) (width 0.2) (layer "F.Cu") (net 2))
 (segment (start 158.91764 78.65364) (end 160.02 79.756) (width 0.2) (layer "F.Cu") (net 2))
 (segment (start 160.02 79.756) (end 165.1 79.756) (width 0.2) (layer "F.Cu") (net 2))
 (segment (start 157.226 78.65364) (end 158.91764 78.65364) (width 0.2) (layer "F.Cu") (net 2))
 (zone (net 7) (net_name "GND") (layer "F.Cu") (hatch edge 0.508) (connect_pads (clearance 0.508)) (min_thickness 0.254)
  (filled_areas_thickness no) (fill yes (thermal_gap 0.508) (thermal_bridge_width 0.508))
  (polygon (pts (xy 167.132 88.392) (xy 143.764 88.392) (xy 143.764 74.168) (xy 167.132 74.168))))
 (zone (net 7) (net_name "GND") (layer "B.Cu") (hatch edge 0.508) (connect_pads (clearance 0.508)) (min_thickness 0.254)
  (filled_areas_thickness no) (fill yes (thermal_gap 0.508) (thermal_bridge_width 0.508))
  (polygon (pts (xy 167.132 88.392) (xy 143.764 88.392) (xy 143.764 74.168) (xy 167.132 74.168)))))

